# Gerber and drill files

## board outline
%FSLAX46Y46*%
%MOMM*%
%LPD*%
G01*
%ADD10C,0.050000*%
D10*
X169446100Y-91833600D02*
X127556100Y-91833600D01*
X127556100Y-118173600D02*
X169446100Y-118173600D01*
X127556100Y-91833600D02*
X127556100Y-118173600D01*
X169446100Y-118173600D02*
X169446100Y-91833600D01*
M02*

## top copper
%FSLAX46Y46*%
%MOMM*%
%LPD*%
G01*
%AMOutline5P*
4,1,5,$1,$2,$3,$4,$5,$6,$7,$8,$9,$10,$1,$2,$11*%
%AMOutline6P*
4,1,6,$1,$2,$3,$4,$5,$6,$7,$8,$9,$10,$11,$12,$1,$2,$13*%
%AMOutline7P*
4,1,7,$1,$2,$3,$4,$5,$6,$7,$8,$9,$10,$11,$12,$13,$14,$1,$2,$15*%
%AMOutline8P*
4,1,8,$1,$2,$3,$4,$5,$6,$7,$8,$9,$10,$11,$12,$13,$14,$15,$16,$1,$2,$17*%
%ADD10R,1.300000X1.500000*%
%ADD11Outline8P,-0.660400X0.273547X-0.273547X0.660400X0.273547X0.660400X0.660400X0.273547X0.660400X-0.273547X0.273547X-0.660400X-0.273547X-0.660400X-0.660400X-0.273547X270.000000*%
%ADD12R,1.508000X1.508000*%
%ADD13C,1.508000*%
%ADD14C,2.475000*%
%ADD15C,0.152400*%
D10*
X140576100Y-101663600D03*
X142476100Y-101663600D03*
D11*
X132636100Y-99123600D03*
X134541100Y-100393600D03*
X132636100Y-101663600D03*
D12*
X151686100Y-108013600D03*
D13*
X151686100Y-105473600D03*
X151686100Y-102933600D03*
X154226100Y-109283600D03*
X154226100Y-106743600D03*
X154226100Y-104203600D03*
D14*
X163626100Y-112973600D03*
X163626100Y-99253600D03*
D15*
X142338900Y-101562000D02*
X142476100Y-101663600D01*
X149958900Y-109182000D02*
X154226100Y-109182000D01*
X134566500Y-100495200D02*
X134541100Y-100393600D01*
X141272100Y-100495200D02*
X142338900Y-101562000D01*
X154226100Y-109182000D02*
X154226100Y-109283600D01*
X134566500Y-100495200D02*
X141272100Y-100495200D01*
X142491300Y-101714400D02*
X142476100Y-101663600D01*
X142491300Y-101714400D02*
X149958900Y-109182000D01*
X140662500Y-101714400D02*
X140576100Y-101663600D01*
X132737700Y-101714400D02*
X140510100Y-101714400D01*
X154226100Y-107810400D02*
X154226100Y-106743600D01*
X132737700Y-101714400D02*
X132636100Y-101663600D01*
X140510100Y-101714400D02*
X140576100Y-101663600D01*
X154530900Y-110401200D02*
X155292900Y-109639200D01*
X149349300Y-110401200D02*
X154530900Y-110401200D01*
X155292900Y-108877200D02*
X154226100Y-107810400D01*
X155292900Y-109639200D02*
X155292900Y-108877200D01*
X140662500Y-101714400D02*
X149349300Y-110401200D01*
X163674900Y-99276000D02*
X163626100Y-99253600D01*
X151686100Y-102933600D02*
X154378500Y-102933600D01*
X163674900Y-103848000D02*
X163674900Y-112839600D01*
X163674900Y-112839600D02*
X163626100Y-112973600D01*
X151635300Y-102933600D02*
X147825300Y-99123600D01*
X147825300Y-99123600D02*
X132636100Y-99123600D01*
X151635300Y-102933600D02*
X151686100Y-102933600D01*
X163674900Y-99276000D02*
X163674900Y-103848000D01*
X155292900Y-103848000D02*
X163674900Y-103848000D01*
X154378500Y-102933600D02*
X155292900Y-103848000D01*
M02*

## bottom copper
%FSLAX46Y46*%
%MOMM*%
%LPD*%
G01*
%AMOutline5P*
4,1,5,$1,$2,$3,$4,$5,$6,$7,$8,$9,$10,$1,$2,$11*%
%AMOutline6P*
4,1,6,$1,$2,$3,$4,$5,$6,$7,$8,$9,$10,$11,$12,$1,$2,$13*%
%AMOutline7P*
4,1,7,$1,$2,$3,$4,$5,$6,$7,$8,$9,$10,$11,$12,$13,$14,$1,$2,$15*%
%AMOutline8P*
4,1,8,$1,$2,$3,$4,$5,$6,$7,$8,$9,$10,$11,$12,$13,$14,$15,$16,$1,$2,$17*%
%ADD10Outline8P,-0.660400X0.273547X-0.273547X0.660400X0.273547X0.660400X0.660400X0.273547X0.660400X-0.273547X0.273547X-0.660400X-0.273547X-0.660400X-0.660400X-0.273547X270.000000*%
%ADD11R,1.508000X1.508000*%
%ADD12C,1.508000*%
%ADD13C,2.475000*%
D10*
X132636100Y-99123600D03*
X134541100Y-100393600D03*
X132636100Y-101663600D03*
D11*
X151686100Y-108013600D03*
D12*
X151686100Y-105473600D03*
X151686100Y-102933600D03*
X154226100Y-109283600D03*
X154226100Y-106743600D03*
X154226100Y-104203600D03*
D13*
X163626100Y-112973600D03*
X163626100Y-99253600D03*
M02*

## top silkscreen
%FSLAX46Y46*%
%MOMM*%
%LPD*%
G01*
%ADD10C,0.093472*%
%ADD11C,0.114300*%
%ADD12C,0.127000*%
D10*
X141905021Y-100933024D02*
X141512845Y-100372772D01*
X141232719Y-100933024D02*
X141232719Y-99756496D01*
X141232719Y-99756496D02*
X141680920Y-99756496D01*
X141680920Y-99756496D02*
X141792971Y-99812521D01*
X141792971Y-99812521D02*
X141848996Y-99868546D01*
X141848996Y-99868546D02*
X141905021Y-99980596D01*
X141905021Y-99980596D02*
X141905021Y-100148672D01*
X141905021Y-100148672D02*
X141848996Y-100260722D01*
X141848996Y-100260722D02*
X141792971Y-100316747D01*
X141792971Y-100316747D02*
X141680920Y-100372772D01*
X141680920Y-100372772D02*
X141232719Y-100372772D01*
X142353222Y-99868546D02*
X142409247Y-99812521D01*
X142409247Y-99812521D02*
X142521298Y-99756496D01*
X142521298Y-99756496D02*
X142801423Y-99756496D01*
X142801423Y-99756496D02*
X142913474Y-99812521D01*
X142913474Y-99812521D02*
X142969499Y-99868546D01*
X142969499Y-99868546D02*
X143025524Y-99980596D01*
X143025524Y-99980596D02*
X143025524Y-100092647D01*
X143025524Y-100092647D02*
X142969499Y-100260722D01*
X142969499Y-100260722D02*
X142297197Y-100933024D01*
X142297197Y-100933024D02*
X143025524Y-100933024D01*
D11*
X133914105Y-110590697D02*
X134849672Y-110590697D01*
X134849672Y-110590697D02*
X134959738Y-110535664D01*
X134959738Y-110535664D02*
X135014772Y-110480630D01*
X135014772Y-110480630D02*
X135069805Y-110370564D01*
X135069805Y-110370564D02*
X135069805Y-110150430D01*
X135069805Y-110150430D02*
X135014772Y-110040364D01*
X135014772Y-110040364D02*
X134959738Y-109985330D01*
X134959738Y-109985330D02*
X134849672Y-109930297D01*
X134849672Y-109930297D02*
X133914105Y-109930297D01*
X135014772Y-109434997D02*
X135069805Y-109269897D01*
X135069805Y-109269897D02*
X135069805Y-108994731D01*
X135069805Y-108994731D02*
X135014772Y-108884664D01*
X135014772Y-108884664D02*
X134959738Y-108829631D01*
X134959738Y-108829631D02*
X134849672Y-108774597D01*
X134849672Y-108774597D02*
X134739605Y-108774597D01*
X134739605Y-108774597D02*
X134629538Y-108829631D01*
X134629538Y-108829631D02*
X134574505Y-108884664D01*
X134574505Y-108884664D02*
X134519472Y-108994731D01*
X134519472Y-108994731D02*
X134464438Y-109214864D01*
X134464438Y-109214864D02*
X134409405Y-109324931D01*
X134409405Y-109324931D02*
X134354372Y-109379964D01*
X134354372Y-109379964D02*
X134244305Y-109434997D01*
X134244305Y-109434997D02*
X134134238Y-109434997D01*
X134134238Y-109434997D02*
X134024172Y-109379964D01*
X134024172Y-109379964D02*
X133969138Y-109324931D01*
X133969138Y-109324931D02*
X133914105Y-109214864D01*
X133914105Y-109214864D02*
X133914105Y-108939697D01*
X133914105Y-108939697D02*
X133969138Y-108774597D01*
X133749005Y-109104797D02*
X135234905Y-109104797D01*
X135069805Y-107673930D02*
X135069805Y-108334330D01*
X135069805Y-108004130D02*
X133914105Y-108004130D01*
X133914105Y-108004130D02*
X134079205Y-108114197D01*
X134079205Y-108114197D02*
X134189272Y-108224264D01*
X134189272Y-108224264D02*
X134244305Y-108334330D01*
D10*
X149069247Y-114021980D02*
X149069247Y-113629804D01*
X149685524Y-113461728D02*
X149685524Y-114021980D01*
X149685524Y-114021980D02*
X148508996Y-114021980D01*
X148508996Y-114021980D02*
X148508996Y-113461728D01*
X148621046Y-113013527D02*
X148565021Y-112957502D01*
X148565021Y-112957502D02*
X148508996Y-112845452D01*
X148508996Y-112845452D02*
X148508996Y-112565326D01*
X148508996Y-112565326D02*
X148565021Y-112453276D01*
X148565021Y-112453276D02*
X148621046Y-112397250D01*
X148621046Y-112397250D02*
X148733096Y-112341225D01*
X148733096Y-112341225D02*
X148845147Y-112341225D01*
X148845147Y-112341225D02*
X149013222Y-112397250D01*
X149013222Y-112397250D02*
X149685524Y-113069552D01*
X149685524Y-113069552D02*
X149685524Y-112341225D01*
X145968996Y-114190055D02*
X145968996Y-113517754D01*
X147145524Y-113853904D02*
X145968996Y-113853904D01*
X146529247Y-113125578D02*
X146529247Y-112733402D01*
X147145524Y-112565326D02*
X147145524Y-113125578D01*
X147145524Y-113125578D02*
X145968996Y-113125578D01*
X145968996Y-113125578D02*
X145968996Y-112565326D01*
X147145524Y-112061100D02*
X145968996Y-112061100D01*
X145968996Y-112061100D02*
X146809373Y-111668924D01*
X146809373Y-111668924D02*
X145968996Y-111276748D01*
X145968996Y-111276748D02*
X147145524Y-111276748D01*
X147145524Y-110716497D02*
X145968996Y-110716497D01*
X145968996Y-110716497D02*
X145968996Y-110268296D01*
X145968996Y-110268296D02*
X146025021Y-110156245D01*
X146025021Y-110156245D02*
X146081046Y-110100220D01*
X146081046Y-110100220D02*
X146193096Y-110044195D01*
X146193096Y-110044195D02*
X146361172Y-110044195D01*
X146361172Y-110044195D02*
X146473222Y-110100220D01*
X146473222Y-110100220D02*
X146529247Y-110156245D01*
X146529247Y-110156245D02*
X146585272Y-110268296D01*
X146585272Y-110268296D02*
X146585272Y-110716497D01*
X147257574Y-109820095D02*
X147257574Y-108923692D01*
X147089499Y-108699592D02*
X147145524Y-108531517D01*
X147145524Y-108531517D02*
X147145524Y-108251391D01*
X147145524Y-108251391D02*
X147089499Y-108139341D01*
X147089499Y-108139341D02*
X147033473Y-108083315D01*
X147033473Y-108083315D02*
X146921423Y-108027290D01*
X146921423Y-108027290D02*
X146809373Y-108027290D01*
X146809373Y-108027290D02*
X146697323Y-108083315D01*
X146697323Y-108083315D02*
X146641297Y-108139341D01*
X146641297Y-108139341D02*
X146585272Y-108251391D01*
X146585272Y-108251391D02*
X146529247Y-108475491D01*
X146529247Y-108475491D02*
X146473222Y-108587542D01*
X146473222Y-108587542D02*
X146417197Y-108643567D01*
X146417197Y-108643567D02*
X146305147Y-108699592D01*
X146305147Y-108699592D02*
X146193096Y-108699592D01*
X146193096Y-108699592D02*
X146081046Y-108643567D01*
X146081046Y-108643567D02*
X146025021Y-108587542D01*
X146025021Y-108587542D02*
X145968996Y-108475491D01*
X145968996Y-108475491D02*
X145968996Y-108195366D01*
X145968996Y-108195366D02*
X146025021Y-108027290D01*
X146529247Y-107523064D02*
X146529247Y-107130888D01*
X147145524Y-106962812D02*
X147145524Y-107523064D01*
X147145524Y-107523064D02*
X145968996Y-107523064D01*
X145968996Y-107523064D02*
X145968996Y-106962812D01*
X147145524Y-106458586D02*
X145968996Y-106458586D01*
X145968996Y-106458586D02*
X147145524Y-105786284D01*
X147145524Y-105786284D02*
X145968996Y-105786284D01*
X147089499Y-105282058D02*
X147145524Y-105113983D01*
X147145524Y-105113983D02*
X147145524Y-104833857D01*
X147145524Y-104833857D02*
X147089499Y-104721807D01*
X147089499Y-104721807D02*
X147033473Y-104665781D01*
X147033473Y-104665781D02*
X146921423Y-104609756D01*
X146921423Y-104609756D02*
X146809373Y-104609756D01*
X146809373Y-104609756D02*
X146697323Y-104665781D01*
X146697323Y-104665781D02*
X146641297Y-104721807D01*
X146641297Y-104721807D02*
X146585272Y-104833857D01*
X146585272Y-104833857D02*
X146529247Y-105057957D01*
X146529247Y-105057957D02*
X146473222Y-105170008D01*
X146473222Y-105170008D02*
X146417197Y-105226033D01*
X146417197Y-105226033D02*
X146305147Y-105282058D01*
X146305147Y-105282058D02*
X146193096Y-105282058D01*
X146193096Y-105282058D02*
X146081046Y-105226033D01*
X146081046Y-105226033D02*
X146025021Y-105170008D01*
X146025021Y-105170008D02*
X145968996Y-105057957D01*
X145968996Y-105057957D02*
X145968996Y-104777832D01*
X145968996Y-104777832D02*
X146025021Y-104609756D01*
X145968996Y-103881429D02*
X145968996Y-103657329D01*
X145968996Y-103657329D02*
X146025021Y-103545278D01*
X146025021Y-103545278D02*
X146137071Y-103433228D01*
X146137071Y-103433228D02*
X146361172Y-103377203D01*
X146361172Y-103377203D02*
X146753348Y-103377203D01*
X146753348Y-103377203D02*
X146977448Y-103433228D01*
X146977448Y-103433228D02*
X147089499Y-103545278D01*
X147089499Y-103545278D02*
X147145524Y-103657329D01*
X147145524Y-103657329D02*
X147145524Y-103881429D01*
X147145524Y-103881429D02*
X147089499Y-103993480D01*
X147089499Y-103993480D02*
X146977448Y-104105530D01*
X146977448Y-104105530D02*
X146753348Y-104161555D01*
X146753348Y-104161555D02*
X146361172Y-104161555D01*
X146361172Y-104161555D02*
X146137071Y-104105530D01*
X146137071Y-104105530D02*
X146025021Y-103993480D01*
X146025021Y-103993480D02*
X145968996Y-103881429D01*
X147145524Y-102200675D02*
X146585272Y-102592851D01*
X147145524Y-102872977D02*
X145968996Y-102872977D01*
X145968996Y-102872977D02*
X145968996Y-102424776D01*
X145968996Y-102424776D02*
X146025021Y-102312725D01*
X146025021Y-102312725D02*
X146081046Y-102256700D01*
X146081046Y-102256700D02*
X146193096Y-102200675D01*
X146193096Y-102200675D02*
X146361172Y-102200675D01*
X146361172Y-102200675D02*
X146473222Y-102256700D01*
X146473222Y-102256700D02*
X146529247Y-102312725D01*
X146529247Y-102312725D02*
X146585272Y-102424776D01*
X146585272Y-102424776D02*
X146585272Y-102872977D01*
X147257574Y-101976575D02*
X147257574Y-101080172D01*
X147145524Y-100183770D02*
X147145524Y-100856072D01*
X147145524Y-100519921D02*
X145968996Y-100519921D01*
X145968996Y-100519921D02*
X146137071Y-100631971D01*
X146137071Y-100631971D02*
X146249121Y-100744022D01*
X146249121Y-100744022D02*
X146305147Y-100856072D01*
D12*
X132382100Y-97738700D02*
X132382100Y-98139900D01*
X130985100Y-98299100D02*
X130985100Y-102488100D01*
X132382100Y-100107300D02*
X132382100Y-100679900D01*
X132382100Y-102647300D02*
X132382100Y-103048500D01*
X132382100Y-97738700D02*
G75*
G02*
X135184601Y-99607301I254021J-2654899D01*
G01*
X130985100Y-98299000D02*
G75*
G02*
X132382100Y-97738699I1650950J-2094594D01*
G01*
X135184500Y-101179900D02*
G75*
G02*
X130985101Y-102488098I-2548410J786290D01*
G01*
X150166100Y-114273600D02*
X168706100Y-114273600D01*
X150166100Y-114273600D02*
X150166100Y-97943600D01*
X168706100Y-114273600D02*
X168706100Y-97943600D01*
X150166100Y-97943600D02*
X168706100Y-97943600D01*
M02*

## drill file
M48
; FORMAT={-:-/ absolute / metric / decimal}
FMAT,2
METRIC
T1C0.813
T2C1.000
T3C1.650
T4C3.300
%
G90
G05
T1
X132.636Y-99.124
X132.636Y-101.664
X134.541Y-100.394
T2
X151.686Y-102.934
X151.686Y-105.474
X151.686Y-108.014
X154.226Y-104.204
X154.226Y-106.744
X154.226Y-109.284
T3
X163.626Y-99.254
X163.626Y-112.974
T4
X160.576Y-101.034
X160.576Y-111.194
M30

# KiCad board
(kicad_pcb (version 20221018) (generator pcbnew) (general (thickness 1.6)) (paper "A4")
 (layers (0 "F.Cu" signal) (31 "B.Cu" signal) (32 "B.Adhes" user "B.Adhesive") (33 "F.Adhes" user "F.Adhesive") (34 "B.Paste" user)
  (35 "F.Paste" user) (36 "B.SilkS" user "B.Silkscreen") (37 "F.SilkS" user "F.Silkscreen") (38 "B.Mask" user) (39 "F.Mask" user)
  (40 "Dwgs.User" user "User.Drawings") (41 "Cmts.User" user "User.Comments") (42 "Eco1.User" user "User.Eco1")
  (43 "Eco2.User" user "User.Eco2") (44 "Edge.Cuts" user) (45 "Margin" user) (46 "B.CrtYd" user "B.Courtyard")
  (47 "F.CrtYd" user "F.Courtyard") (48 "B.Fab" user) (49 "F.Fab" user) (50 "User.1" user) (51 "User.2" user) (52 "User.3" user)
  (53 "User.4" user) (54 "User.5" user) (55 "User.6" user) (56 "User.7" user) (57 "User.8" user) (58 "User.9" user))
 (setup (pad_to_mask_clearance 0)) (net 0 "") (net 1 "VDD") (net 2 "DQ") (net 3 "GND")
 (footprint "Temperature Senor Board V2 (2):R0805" (layer "F.Cu") (at 141.5261 101.6636)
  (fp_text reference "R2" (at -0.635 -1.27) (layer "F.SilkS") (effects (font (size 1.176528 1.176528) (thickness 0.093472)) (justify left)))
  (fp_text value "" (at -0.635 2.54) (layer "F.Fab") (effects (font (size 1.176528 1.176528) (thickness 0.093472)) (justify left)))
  (pad "1" smd rect (at -0.95 0) (size 1.3 1.5) (layers "F.Cu" "F.Paste" "F.Mask") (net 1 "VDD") (solder_mask_margin 0.1016)
   (thermal_bridge_angle 45))
  (pad "2" smd rect (at 0.95 0) (size 1.3 1.5) (layers "F.Cu" "F.Paste" "F.Mask") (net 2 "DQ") (solder_mask_margin 0.1016)
   (thermal_bridge_angle 45)))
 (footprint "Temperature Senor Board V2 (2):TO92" (layer "F.Cu") (at 132.6361 100.3936 -90)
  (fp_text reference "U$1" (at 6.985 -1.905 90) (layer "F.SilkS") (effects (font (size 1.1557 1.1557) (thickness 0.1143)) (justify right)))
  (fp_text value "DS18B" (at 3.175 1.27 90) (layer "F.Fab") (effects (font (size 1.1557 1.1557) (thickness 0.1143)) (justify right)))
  (fp_line (start -2.6549 0.254) (end -2.2537 0.254) (stroke (width 0.127) (type solid)) (layer "F.SilkS"))
  (fp_line (start -2.0945 1.651) (end 2.0945 1.651) (stroke (width 0.127) (type solid)) (layer "F.SilkS"))
  (fp_line (start -0.2863 0.254) (end 0.2863 0.254) (stroke (width 0.127) (type solid)) (layer "F.SilkS"))
  (fp_line (start 2.2537 0.254) (end 2.6549 0.254) (stroke (width 0.127) (type solid)) (layer "F.SilkS"))
  (fp_arc (start -2.6549 0.254) (mid -2.219001 -1.479566) (end -0.786299 -2.548501) (stroke (width 0.127) (type solid)) (layer "F.SilkS"))
  (fp_arc (start -2.0946 1.651) (mid -2.475347 0.992847) (end -2.654901 0.254) (stroke (width 0.127) (type solid)) (layer "F.SilkS"))
  (fp_arc (start 0.7863 -2.5484) (mid 2.546275 -0.793203) (end 2.094499 1.651) (stroke (width 0.127) (type solid)) (layer "F.SilkS"))
  (pad "1" thru_hole roundrect (at -1.27 0 270) (size 1.3208 1.3208) (drill 0.8128) (layers "*.Cu" "*.Mask") (roundrect_rratio 0.25)
   (chamfer_ratio 0.2928932188) (chamfer top_left top_right bottom_left bottom_right) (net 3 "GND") (solder_mask_margin 0.1016)
   (thermal_bridge_angle 45))
  (pad "2" thru_hole roundrect (at 0 -1.905 270) (size 1.3208 1.3208) (drill 0.8128) (layers "*.Cu" "*.Mask") (roundrect_rratio 0.25)
   (chamfer_ratio 0.2928932188) (chamfer top_left top_right bottom_left bottom_right) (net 2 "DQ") (solder_mask_margin 0.1016)
   (thermal_bridge_angle 45))
  (pad "3" thru_hole roundrect (at 1.27 0 270) (size 1.3208 1.3208) (drill 0.8128) (layers "*.Cu" "*.Mask") (roundrect_rratio 0.25)
   (chamfer_ratio 0.2928932188) (chamfer top_left top_right bottom_left bottom_right) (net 1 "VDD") (solder_mask_margin 0.1016)
   (thermal_bridge_angle 45)))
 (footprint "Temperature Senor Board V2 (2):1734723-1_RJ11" (layer "F.Cu") (at 154.2261 105.4736 90)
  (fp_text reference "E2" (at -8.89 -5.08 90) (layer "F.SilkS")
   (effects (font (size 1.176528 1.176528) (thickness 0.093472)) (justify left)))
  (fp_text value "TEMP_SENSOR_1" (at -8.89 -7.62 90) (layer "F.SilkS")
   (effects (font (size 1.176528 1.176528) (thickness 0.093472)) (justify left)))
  (fp_line (start -8.8 -4.06) (end -8.8 14.48) (stroke (width 0.127) (type solid)) (layer "F.SilkS"))
  (fp_line (start -8.8 -4.06) (end 7.53 -4.06) (stroke (width 0.127) (type solid)) (layer "F.SilkS"))
  (fp_line (start -8.8 14.48) (end 7.53 14.48) (stroke (width 0.127) (type solid)) (layer "F.SilkS"))
  (fp_line (start 7.53 -4.06) (end 7.53 14.48) (stroke (width 0.127) (type solid)) (layer "F.SilkS"))
  (pad "" np_thru_hole circle (at -5.72 6.35 90) (size 3.3 3.3) (drill 3.3) (layers "*.Cu" "*.Mask"))
  (pad "" np_thru_hole circle (at 4.44 6.35 90) (size 3.3 3.3) (drill 3.3) (layers "*.Cu" "*.Mask"))
  (pad "1" thru_hole rect (at -2.54 -2.54 90) (size 1.508 1.508) (drill 1) (layers "*.Cu" "*.Mask") (solder_mask_margin 0.1016)
   (thermal_bridge_angle 45))
  (pad "2" thru_hole circle (at 0 -2.54 90) (size 1.508 1.508) (drill 1) (layers "*.Cu" "*.Mask") (solder_mask_margin 0.1016))
  (pad "3" thru_hole circle (at 2.54 -2.54 90) (size 1.508 1.508) (drill 1) (layers "*.Cu" "*.Mask") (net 3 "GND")
   (solder_mask_margin 0.1016))
  (pad "4" thru_hole circle (at -3.81 0 90) (size 1.508 1.508) (drill 1) (layers "*.Cu" "*.Mask") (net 2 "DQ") (solder_mask_margin 0.1016))
  (pad "5" thru_hole circle (at -1.27 0 90) (size 1.508 1.508) (drill 1) (layers "*.Cu" "*.Mask") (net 1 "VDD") (solder_mask_margin 0.1016))
  (pad "6" thru_hole circle (at 1.27 0 90) (size 1.508 1.508) (drill 1) (layers "*.Cu" "*.Mask") (solder_mask_margin 0.1016))
  (pad "SH1" thru_hole circle (at -7.5 9.4 90) (size 2.475 2.475) (drill 1.65) (layers "*.Cu" "*.Mask") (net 3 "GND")
   (solder_mask_margin 0.1016))
  (pad "SH2" thru_hole circle (at 6.22 9.4 90) (size 2.475 2.475) (drill 1.65) (layers "*.Cu" "*.Mask") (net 3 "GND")
   (solder_mask_margin 0.1016)))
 (gr_line (start 169.4461 91.8336) (end 127.5561 91.8336) (stroke (width 0.05) (type solid)) (layer "Edge.Cuts"))
 (gr_line (start 127.5561 118.1736) (end 169.4461 118.1736) (stroke (width 0.05) (type solid)) (layer "Edge.Cuts"))
 (gr_line (start 127.5561 91.8336) (end 127.5561 118.1736) (stroke (width 0.05) (type solid)) (layer "Edge.Cuts"))
 (gr_line (start 169.4461 118.1736) (end 169.4461 91.8336) (stroke (width 0.05) (type solid)) (layer "Edge.Cuts"))
 (segment (start 142.3389 101.562) (end 142.4761 101.6636) (width 0.1524) (layer "F.Cu") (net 2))
 (segment (start 149.9589 109.182) (end 154.2261 109.182) (width 0.1524) (layer "F.Cu") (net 2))
 (segment (start 134.5665 100.4952) (end 134.5411 100.3936) (width 0.1524) (layer "F.Cu") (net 2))
 (segment (start 141.2721 100.4952) (end 142.3389 101.562) (width 0.1524) (layer "F.Cu") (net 2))
 (segment (start 154.2261 109.182) (end 154.2261 109.2836) (width 0.1524) (layer "F.Cu") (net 2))
 (segment (start 134.5665 100.4952) (end 141.2721 100.4952) (width 0.1524) (layer "F.Cu") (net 2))
 (segment (start 142.4913 101.7144) (end 142.4761 101.6636) (width 0.1524) (layer "F.Cu") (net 2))
 (segment (start 142.4913 101.7144) (end 149.9589 109.182) (width 0.1524) (layer "F.Cu") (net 2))
 (segment (start 140.6625 101.7144) (end 140.5761 101.6636) (width 0.1524) (layer "F.Cu") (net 1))
 (segment (start 132.7377 101.7144) (end 140.5101 101.7144) (width 0.1524) (layer "F.Cu") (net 1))
 (segment (start 154.2261 107.8104) (end 154.2261 106.7436) (width 0.1524) (layer "F.Cu") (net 1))
 (segment (start 132.7377 101.7144) (end 132.6361 101.6636) (width 0.1524) (layer "F.Cu") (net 1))
 (segment (start 140.5101 101.7144) (end 140.5761 101.6636) (width 0.1524) (layer "F.Cu") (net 1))
 (segment (start 154.5309 110.4012) (end 155.2929 109.6392) (width 0.1524) (layer "F.Cu") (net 1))
 (segment (start 149.3493 110.4012) (end 154.5309 110.4012) (width 0.1524) (layer "F.Cu") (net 1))
 (segment (start 155.2929 108.8772) (end 154.2261 107.8104) (width 0.1524) (layer "F.Cu") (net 1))
 (segment (start 155.2929 109.6392) (end 155.2929 108.8772) (width 0.1524) (layer "F.Cu") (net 1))
 (segment (start 140.6625 101.7144) (end 149.3493 110.4012) (width 0.1524) (layer "F.Cu") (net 1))
 (segment (start 163.6749 99.276) (end 163.6261 99.2536) (width 0.1524) (layer "F.Cu") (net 3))
 (segment (start 151.6861 102.9336) (end 154.3785 102.9336) (width 0.1524) (layer "F.Cu") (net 3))
 (segment (start 163.6749 103.848) (end 163.6749 112.8396) (width 0.1524) (layer "F.Cu") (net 3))
 (segment (start 163.6749 112.8396) (end 163.6261 112.9736) (width 0.1524) (layer "F.Cu") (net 3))
 (segment (start 151.6353 102.9336) (end 147.8253 99.1236) (width 0.1524) (layer "F.Cu") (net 3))
 (segment (start 147.8253 99.1236) (end 132.6361 99.1236) (width 0.1524) (layer "F.Cu") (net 3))
 (segment (start 151.6353 102.9336) (end 151.6861 102.9336) (width 0.1524) (layer "F.Cu") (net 3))
 (segment (start 163.6749 99.276) (end 163.6749 103.848) (width 0.1524) (layer "F.Cu") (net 3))
 (segment (start 155.2929 103.848) (end 163.6749 103.848) (width 0.1524) (layer "F.Cu") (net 3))
 (segment (start 154.3785 102.9336) (end 155.2929 103.848) (width 0.1524) (layer "F.Cu") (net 3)))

